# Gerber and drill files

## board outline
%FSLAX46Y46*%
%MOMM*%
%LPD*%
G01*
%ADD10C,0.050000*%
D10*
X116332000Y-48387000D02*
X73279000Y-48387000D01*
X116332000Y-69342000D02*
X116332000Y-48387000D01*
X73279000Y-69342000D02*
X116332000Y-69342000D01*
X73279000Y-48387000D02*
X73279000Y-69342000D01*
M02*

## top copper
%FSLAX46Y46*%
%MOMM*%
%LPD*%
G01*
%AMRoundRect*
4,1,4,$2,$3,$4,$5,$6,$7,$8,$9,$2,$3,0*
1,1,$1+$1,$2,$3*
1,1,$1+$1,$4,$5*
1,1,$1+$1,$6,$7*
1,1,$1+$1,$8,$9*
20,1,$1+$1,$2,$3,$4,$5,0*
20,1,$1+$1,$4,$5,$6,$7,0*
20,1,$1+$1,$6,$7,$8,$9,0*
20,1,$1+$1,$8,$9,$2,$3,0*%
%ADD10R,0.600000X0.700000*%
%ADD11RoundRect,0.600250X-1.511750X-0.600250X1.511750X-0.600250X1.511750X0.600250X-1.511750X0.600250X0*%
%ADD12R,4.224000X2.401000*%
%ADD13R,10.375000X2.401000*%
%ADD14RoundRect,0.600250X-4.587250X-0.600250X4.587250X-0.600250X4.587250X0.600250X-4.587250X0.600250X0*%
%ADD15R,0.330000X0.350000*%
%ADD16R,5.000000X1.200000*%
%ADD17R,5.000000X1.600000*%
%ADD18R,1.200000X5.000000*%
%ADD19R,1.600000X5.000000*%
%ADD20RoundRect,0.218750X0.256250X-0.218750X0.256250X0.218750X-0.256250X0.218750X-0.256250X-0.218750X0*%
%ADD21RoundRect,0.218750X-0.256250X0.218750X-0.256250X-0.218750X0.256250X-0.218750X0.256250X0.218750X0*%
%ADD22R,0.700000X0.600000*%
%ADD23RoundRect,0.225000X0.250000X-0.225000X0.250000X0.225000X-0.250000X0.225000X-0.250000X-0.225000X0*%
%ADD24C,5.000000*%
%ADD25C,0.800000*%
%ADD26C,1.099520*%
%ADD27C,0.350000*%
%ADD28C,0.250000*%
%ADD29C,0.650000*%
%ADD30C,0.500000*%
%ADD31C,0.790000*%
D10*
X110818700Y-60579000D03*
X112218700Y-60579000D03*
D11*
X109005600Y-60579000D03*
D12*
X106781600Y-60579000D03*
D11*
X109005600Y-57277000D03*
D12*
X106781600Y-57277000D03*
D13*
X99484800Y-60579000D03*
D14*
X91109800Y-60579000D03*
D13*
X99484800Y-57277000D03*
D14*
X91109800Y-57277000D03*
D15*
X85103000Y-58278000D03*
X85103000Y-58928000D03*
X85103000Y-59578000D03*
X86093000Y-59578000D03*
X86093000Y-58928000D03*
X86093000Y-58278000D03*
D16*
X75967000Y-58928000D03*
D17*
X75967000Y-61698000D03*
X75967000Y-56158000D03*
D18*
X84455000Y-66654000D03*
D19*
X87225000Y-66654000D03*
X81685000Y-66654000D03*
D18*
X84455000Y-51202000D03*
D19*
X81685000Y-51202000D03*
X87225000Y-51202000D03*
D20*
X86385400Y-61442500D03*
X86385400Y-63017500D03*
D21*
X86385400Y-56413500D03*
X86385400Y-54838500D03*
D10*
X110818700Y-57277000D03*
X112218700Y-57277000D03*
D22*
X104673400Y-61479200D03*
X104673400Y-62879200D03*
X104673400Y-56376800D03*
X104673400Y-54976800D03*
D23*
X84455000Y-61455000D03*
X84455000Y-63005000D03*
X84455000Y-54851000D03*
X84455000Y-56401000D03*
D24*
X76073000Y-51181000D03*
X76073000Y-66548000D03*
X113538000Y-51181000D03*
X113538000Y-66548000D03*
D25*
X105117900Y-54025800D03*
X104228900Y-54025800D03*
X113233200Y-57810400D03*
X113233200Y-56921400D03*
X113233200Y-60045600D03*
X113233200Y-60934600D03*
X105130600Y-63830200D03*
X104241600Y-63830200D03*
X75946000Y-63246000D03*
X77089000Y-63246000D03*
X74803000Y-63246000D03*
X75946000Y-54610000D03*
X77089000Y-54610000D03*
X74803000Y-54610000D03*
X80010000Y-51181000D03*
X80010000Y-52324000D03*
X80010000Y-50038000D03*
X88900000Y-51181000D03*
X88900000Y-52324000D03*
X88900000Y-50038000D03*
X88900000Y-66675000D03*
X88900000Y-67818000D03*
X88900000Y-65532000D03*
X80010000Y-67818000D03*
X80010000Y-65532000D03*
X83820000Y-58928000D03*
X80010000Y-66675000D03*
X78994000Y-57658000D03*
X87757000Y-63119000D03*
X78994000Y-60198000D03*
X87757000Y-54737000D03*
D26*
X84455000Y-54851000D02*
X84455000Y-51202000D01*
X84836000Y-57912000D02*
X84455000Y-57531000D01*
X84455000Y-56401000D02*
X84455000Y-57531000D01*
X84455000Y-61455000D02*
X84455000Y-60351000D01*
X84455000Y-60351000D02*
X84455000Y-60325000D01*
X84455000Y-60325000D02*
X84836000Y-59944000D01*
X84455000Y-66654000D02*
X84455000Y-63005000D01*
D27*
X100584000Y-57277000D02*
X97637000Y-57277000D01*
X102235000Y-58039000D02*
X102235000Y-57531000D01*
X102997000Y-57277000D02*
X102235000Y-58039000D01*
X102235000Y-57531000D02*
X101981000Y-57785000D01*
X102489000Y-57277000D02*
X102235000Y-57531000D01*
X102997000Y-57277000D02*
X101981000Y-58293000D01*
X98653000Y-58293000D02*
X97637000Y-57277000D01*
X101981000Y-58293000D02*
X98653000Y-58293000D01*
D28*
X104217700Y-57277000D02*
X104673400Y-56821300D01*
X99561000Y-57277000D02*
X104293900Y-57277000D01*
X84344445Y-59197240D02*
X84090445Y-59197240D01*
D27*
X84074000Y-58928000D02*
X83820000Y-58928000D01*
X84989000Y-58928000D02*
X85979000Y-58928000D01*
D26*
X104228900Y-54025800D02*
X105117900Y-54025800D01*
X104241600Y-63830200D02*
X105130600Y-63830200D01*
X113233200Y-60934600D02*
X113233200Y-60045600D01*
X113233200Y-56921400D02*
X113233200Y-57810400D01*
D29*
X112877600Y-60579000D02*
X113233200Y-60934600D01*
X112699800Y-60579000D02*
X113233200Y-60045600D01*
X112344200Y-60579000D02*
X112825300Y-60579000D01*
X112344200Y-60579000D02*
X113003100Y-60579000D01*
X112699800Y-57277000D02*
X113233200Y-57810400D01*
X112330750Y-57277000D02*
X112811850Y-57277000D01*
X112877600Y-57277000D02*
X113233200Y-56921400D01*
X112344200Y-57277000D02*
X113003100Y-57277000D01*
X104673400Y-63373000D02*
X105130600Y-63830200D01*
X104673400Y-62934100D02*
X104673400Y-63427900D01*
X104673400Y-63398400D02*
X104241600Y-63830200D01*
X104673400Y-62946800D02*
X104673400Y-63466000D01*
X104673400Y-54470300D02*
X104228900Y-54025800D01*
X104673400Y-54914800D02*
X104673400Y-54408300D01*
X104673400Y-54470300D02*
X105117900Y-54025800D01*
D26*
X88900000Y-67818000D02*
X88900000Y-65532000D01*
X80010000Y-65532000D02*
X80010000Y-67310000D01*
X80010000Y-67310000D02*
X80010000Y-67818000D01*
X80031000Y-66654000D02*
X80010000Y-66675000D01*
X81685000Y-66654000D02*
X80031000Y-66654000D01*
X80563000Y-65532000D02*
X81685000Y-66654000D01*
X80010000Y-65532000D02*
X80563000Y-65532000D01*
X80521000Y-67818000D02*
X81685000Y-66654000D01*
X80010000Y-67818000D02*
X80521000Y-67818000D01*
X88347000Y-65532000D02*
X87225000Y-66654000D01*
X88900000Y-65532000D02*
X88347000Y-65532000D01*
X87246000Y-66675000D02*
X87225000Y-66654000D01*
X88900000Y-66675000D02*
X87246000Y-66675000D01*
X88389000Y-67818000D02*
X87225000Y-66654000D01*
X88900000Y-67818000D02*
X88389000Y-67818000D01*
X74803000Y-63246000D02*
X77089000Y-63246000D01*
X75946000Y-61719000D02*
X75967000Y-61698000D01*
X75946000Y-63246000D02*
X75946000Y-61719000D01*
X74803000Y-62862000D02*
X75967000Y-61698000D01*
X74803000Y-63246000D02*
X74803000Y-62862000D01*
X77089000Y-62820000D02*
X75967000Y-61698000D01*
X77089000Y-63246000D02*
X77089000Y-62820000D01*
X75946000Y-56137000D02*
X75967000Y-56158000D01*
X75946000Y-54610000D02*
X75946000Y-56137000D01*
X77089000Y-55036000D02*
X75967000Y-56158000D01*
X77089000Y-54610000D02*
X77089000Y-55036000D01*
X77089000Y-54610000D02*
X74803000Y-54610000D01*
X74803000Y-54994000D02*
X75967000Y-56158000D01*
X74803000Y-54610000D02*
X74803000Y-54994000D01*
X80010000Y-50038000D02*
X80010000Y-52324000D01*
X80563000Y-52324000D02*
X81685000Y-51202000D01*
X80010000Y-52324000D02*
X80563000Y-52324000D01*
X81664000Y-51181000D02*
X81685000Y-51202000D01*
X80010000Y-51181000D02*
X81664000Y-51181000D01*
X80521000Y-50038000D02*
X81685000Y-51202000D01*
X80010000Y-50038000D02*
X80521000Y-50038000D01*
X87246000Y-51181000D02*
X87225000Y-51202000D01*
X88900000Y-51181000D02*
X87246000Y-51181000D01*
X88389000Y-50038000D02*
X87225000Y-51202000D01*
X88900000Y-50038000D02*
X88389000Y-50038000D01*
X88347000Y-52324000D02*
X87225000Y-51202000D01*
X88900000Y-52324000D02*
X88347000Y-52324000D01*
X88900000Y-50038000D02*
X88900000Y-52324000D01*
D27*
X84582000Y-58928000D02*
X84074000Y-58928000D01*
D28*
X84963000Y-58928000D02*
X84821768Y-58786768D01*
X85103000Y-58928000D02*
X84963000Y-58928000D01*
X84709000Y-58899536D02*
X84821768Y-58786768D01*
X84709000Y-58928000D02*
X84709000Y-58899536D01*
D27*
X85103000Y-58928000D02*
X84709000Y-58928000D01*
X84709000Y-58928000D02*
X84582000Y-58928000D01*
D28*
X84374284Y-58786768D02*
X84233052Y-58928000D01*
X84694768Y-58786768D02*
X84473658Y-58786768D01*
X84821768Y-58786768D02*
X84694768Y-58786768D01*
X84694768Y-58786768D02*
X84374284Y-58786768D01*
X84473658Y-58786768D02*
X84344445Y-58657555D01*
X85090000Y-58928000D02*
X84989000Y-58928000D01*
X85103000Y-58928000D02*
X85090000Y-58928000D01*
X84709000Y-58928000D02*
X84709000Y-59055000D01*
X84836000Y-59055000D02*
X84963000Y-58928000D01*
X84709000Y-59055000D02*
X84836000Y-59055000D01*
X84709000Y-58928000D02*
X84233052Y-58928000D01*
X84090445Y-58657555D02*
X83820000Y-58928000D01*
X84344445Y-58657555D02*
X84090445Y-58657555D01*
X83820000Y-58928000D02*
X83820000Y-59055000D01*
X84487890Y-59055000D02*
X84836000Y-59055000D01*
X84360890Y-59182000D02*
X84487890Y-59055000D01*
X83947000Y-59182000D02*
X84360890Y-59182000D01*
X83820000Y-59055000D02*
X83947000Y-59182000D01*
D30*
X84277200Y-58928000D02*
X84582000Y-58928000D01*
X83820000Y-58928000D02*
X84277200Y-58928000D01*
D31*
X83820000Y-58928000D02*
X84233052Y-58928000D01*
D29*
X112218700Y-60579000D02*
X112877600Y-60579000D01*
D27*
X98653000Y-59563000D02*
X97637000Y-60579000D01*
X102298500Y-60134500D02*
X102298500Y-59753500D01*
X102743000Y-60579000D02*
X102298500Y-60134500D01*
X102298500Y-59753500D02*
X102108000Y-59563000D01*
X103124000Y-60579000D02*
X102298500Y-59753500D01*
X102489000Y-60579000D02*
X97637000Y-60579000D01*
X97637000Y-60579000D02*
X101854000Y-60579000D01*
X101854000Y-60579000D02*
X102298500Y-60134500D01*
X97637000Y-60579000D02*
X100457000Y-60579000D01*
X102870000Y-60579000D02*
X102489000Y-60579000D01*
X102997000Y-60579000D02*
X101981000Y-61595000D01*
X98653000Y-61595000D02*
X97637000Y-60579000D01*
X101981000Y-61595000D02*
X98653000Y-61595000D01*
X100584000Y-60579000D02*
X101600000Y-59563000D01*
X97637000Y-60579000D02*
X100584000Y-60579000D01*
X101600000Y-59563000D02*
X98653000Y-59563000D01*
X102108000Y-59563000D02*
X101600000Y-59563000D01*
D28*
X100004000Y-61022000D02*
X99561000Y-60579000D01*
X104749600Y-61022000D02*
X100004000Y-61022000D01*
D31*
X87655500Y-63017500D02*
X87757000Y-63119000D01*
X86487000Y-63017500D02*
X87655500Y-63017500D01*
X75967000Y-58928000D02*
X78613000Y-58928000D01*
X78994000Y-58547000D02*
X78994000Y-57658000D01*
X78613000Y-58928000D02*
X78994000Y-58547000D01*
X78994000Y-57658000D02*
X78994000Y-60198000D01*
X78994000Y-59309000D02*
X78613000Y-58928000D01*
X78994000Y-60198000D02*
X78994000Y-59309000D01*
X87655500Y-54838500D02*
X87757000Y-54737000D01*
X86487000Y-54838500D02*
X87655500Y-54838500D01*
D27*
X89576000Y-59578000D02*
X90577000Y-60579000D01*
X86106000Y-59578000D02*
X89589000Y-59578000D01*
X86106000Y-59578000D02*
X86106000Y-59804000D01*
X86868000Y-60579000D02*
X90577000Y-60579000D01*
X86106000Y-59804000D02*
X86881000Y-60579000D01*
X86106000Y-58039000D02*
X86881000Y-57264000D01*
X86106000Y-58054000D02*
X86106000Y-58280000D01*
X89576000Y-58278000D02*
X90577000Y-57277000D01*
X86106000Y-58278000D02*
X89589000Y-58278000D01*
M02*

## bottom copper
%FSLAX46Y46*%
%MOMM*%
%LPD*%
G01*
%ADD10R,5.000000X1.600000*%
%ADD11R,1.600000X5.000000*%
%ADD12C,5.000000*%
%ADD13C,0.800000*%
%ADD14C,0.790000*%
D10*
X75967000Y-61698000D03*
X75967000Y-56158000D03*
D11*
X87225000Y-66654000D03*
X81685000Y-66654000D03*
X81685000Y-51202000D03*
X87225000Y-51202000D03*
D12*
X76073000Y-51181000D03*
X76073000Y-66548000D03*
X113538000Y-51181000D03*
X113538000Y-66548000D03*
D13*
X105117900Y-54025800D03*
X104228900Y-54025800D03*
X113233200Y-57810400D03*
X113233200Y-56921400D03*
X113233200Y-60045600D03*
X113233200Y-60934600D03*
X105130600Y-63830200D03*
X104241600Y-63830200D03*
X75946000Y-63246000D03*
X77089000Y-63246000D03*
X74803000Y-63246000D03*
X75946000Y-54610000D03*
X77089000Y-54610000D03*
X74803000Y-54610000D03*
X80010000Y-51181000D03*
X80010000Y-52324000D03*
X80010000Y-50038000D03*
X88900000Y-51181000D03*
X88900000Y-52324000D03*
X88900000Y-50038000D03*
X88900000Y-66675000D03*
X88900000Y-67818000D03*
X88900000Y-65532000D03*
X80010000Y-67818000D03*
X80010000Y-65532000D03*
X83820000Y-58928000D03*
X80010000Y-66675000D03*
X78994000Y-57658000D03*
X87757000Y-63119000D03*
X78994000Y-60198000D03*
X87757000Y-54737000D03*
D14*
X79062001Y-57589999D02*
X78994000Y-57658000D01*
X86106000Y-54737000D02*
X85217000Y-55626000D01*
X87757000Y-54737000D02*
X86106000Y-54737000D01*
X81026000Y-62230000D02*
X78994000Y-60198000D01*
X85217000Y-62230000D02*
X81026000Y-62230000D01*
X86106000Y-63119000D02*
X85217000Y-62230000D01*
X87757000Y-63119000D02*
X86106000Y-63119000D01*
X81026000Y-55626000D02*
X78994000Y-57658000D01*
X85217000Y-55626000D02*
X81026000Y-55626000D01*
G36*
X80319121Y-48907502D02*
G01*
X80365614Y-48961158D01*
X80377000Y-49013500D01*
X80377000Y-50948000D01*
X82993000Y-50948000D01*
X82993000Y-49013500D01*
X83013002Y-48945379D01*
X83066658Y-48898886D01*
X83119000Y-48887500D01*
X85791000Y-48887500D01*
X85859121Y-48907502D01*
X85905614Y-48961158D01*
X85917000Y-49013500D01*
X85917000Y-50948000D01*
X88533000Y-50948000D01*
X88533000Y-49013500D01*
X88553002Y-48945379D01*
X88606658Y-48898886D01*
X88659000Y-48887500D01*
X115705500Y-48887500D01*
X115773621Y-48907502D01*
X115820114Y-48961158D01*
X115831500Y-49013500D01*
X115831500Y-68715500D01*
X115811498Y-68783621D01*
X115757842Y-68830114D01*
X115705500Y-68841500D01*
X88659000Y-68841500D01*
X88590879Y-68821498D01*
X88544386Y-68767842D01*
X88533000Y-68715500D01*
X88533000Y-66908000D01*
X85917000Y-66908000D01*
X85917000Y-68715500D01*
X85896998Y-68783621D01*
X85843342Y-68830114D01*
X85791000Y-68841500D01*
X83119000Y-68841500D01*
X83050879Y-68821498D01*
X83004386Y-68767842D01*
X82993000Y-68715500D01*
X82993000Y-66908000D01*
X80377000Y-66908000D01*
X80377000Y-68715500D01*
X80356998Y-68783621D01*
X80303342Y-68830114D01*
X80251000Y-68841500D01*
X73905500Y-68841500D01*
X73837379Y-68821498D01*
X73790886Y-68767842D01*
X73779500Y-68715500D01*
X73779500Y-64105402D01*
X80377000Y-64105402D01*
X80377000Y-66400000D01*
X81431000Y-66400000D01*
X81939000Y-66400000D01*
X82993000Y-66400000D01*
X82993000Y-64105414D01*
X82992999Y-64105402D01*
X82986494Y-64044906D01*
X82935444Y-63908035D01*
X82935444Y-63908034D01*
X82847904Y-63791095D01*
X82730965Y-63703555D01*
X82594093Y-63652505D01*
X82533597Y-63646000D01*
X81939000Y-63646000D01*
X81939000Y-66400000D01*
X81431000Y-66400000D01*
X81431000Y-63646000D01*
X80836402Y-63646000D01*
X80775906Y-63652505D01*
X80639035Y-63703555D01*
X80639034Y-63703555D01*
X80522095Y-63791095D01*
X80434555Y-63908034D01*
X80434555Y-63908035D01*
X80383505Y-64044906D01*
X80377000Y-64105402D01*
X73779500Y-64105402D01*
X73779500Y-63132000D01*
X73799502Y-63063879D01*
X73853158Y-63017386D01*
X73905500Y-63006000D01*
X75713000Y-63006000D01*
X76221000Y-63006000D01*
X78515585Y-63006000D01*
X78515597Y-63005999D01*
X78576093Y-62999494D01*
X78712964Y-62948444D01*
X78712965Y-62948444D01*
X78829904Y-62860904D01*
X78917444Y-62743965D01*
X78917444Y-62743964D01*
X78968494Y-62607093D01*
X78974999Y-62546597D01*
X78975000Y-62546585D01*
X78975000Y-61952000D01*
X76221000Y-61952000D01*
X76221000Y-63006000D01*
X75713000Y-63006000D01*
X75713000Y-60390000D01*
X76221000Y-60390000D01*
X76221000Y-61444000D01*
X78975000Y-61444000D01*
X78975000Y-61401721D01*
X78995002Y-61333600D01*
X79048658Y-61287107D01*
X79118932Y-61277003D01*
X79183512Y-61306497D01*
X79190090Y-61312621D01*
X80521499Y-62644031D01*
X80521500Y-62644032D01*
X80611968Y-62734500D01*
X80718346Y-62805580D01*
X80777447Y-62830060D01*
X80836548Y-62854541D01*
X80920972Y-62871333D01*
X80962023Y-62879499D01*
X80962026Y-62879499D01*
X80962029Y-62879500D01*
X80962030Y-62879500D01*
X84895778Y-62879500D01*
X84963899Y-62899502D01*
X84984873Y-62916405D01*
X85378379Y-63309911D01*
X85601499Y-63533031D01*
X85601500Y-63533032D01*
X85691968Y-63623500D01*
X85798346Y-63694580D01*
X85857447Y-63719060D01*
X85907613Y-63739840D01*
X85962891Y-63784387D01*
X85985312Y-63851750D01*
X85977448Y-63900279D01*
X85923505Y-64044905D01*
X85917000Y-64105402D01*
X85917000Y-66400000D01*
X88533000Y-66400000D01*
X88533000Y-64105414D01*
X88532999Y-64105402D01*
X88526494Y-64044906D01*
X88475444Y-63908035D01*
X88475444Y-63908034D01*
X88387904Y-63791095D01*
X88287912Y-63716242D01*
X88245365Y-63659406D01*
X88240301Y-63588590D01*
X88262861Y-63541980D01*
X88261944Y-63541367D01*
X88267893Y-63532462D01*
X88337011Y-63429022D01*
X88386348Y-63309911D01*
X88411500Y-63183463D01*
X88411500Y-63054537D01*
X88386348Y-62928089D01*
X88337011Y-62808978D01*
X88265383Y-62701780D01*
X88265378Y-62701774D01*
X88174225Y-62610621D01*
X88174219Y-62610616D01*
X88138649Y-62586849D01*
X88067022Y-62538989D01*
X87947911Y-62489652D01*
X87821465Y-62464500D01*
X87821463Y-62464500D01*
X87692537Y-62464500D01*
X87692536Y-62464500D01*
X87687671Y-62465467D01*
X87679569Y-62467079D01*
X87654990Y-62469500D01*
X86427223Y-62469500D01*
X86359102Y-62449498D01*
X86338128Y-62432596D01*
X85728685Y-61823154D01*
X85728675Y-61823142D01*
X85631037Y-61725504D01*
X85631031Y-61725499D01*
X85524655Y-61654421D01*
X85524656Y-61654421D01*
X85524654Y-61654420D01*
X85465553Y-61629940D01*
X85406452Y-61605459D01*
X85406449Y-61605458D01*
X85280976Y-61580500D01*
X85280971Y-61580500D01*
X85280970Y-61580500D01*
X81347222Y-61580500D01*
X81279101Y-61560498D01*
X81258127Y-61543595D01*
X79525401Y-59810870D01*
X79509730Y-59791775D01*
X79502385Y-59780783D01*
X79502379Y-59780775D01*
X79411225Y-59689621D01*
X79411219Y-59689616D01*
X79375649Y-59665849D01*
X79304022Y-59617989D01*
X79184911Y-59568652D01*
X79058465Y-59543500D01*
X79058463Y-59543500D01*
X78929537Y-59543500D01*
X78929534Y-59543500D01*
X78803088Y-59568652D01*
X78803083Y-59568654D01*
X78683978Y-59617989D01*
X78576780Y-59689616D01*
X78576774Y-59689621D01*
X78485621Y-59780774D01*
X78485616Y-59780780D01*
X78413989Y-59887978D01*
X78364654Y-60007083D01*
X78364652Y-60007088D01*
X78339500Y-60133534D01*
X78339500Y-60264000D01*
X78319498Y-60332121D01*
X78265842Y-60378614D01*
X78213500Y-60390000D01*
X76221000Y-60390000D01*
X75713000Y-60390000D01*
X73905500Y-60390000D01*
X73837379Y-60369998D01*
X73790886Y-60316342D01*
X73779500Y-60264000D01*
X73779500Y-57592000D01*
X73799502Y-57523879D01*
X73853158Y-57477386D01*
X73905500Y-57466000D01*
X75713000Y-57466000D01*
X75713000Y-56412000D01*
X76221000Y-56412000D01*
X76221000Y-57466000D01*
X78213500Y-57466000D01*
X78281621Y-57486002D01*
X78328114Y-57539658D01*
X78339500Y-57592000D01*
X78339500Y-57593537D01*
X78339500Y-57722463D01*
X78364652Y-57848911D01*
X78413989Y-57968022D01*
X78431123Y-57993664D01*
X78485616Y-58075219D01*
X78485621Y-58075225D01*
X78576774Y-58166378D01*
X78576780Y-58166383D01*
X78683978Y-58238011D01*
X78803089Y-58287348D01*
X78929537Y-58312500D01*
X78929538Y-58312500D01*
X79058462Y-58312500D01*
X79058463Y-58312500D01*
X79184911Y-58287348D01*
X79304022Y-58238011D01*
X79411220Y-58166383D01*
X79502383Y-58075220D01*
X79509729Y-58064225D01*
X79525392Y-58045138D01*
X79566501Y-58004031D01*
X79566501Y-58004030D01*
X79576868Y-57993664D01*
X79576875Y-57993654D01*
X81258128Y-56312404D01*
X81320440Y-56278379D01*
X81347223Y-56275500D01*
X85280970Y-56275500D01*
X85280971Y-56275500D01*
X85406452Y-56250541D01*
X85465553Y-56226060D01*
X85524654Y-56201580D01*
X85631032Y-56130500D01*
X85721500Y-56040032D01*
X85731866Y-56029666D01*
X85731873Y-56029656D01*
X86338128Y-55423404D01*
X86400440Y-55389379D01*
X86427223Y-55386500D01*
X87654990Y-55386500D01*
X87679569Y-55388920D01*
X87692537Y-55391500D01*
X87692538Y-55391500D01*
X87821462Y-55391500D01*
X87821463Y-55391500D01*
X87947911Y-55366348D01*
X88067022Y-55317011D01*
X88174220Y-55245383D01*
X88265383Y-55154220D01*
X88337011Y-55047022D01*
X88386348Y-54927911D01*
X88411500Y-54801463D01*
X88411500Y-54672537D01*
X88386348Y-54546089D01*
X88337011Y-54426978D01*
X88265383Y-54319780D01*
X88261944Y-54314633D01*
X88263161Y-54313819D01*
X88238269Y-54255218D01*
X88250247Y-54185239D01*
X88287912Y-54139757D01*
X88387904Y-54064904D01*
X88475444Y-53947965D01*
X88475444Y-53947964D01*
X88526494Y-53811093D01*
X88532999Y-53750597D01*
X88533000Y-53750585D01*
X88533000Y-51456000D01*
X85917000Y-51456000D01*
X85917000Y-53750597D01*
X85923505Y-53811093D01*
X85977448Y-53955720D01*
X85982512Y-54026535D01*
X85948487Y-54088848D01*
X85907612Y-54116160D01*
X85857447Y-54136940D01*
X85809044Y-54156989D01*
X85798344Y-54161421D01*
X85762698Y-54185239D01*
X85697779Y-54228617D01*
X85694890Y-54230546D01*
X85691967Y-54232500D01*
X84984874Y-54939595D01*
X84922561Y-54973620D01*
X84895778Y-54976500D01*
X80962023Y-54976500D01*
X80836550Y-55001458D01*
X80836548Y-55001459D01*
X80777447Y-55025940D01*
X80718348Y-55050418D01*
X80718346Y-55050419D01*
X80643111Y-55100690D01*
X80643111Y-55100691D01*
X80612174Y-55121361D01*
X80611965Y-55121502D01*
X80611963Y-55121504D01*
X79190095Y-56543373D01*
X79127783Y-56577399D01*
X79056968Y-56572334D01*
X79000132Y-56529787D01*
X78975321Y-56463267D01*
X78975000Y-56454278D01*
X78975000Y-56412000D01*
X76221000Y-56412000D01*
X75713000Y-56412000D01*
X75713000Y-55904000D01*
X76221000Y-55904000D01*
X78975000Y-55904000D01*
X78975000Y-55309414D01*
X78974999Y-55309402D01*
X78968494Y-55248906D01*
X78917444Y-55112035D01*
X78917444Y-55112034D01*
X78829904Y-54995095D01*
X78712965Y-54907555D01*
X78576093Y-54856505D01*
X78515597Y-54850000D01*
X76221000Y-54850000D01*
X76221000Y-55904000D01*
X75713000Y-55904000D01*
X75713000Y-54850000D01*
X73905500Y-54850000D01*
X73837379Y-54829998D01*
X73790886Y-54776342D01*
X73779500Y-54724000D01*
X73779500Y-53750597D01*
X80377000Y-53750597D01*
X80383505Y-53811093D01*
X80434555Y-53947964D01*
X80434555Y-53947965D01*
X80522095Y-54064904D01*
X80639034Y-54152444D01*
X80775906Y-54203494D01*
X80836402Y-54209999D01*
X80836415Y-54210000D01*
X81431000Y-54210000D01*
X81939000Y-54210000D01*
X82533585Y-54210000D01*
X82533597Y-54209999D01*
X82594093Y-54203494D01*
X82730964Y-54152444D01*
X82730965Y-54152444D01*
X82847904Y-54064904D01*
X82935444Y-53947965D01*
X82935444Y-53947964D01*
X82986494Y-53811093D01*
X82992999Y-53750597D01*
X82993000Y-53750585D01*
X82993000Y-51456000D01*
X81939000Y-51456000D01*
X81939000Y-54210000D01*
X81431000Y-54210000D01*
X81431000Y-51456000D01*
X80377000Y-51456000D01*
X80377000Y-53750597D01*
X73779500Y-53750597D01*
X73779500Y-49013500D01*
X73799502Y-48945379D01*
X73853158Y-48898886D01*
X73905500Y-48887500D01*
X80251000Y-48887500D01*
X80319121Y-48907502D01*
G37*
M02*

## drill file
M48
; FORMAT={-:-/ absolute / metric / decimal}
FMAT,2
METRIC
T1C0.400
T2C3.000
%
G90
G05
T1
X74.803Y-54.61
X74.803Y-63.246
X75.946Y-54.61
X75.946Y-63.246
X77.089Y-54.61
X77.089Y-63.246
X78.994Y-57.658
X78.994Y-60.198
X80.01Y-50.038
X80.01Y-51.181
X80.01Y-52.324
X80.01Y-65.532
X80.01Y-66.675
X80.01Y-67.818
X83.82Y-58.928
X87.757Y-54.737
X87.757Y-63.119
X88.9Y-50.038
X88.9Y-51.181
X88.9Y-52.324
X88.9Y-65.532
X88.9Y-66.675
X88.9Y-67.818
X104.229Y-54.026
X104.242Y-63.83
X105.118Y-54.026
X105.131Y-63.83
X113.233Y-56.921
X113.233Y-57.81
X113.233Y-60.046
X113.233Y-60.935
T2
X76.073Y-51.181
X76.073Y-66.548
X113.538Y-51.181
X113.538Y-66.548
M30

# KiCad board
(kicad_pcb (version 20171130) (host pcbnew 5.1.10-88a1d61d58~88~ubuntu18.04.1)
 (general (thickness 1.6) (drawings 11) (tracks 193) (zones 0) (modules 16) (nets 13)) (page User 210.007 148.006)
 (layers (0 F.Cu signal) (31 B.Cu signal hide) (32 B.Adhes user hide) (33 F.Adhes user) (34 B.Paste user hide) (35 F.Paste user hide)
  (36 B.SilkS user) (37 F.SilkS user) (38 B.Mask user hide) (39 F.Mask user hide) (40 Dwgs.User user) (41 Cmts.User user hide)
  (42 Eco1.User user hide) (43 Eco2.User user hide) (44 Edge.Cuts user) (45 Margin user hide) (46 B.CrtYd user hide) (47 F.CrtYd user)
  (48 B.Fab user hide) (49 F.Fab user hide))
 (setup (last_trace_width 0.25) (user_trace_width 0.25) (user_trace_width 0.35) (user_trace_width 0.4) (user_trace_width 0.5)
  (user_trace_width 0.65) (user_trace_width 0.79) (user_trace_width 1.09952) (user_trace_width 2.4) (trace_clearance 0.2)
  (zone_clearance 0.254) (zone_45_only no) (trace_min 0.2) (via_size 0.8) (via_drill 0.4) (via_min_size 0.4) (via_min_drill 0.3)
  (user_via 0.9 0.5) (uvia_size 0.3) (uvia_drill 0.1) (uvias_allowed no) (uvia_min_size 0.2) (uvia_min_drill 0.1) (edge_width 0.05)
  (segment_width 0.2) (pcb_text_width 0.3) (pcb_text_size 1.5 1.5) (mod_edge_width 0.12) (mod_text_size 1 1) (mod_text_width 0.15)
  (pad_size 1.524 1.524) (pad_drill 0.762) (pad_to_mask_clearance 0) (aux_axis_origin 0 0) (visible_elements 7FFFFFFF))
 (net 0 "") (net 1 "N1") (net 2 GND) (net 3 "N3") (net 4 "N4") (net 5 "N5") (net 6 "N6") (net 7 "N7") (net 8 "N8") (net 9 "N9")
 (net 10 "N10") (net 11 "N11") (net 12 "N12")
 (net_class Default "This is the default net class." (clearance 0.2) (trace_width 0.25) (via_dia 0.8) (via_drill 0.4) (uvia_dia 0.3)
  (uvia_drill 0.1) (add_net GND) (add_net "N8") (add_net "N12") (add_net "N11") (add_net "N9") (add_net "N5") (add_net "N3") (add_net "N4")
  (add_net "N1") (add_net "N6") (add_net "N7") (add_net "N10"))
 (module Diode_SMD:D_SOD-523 (layer F.Cu) (at 111.5187 60.579)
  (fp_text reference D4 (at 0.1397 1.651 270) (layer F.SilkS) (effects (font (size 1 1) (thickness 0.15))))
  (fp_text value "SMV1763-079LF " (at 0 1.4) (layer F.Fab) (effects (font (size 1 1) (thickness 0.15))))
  (pad 1 smd rect (at -0.7 0 180) (size 0.6 0.7) (layers F.Cu F.Paste F.Mask) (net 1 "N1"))
  (pad 2 smd rect (at 0.7 0 180) (size 0.6 0.7) (layers F.Cu F.Paste F.Mask) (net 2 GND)))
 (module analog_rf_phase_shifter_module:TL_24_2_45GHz (layer F.Cu) (at 107.8936 60.579)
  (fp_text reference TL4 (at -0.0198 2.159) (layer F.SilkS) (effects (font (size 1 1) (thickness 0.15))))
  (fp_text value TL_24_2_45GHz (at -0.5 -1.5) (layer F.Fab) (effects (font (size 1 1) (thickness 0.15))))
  (pad 2 smd roundrect (at 1.112 0) (size 4.224 2.401) (layers F.Cu) (roundrect_rratio 0.25) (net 1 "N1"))
  (pad 1 smd rect (at -1.112 0) (size 4.224 2.401) (layers F.Cu) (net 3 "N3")))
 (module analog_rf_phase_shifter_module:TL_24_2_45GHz (layer F.Cu) (at 107.8936 57.277)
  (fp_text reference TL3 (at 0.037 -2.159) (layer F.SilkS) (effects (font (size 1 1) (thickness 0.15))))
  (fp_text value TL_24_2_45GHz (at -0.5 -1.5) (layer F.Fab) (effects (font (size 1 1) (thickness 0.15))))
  (pad 2 smd roundrect (at 1.112 0) (size 4.224 2.401) (layers F.Cu) (roundrect_rratio 0.25) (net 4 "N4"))
  (pad 1 smd rect (at -1.112 0) (size 4.224 2.401) (layers F.Cu) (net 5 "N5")))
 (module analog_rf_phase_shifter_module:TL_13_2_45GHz (layer F.Cu) (at 95.2973 60.579)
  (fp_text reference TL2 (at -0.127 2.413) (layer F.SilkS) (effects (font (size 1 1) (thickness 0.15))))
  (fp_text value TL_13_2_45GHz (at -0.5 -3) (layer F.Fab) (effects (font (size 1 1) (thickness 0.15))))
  (pad 2 smd rect (at 4.1875 0) (size 10.375 2.401) (layers F.Cu) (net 3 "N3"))
  (pad 1 smd roundrect (at -4.1875 0) (size 10.375 2.401) (layers F.Cu) (roundrect_rratio 0.25) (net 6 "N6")))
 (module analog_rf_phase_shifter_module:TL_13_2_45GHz (layer F.Cu) (at 95.2973 57.277)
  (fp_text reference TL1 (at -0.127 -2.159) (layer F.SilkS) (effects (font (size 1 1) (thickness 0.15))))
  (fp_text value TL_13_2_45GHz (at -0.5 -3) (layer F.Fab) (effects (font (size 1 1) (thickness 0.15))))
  (pad 2 smd rect (at 4.1875 0) (size 10.375 2.401) (layers F.Cu) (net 5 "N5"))
  (pad 1 smd roundrect (at -4.1875 0) (size 10.375 2.401) (layers F.Cu) (roundrect_rratio 0.25) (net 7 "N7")))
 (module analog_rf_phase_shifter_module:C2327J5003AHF (layer F.Cu) (at 85.598 58.928 270)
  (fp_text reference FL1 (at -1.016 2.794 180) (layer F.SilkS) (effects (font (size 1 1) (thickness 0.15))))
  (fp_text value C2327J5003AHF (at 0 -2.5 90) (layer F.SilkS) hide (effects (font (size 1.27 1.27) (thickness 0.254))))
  (pad 1 smd rect (at -0.65 0.495) (size 0.33 0.35) (layers F.Cu F.Paste F.Mask) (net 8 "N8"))
  (pad 2 smd rect (at 0 0.495) (size 0.33 0.35) (layers F.Cu F.Paste F.Mask) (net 2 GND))
  (pad 3 smd rect (at 0.65 0.495) (size 0.33 0.35) (layers F.Cu F.Paste F.Mask) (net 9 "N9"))
  (pad 4 smd rect (at 0.65 -0.495) (size 0.33 0.35) (layers F.Cu F.Paste F.Mask) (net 6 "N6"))
  (pad 5 smd rect (at 0 -0.495) (size 0.33 0.35) (layers F.Cu F.Paste F.Mask) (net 2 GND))
  (pad 6 smd rect (at -0.65 -0.495) (size 0.33 0.35) (layers F.Cu F.Paste F.Mask) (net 7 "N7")))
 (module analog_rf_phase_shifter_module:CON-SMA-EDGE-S (layer F.Cu) (at 68.707 58.928 90)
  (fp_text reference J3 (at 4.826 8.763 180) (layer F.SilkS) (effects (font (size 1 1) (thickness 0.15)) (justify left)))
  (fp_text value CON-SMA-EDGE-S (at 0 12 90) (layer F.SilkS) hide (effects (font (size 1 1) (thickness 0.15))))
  (pad 1 smd rect (at 0 7.26 90) (size 1.2 5) (layers F.Cu F.Paste F.Mask) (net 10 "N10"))
  (pad 2 smd rect (at -2.77 7.26 90) (size 1.6 5) (layers F.Cu F.Paste F.Mask) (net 2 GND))
  (pad 2 smd rect (at 2.77 7.26 90) (size 1.6 5) (layers F.Cu F.Paste F.Mask) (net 2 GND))
  (pad 2 smd rect (at -2.77 7.26 90) (size 1.6 5) (layers B.Cu B.Paste B.Mask) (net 2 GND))
  (pad 2 smd rect (at 2.77 7.26 90) (size 1.6 5) (layers B.Cu B.Paste B.Mask) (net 2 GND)))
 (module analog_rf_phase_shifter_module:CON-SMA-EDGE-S (layer F.Cu) (at 84.455 73.914 180)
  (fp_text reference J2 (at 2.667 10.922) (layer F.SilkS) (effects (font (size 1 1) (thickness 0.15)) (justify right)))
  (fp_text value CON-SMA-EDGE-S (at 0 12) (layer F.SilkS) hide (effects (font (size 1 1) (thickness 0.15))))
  (pad 1 smd rect (at 0 7.26 180) (size 1.2 5) (layers F.Cu F.Paste F.Mask) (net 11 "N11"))
  (pad 2 smd rect (at -2.77 7.26 180) (size 1.6 5) (layers F.Cu F.Paste F.Mask) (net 2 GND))
  (pad 2 smd rect (at 2.77 7.26 180) (size 1.6 5) (layers F.Cu F.Paste F.Mask) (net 2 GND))
  (pad 2 smd rect (at -2.77 7.26 180) (size 1.6 5) (layers B.Cu B.Paste B.Mask) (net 2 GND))
  (pad 2 smd rect (at 2.77 7.26 180) (size 1.6 5) (layers B.Cu B.Paste B.Mask) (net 2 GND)))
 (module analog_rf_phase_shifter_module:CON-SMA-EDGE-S (layer F.Cu) (at 84.455 43.942)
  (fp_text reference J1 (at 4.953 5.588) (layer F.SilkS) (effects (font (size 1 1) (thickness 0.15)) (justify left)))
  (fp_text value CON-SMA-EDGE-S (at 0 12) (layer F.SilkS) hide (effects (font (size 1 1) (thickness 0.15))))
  (pad 1 smd rect (at 0 7.26) (size 1.2 5) (layers F.Cu F.Paste F.Mask) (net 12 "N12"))
  (pad 2 smd rect (at -2.77 7.26) (size 1.6 5) (layers F.Cu F.Paste F.Mask) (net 2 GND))
  (pad 2 smd rect (at 2.77 7.26) (size 1.6 5) (layers F.Cu F.Paste F.Mask) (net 2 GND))
  (pad 2 smd rect (at -2.77 7.26) (size 1.6 5) (layers B.Cu B.Paste B.Mask) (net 2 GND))
  (pad 2 smd rect (at 2.77 7.26) (size 1.6 5) (layers B.Cu B.Paste B.Mask) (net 2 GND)))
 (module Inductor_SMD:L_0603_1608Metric (layer F.Cu) (at 86.3854 62.23 90)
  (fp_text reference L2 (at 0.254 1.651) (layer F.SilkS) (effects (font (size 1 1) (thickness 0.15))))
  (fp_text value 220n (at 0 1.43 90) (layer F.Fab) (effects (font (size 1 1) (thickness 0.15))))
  (pad 2 smd roundrect (at 0.7875 0 90) (size 0.875 0.95) (layers F.Cu F.Paste F.Mask) (roundrect_rratio 0.25) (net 6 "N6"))
  (pad 1 smd roundrect (at -0.7875 0 90) (size 0.875 0.95) (layers F.Cu F.Paste F.Mask) (roundrect_rratio 0.25) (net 10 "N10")))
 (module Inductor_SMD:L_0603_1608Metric (layer F.Cu) (at 86.3854 55.626 270)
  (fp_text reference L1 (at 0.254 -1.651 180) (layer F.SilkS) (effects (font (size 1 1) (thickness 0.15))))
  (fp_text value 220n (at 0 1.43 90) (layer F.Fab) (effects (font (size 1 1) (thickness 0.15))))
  (pad 2 smd roundrect (at 0.7875 0 270) (size 0.875 0.95) (layers F.Cu F.Paste F.Mask) (roundrect_rratio 0.25) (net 7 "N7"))
  (pad 1 smd roundrect (at -0.7875 0 270) (size 0.875 0.95) (layers F.Cu F.Paste F.Mask) (roundrect_rratio 0.25) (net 10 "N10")))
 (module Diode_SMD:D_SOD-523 (layer F.Cu) (at 111.5187 57.277)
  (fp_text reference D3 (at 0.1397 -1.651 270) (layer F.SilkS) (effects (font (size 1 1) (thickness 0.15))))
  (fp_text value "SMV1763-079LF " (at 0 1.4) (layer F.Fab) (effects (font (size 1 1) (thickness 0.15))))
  (pad 1 smd rect (at -0.7 0 180) (size 0.6 0.7) (layers F.Cu F.Paste F.Mask) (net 4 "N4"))
  (pad 2 smd rect (at 0.7 0 180) (size 0.6 0.7) (layers F.Cu F.Paste F.Mask) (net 2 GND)))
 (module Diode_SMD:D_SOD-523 (layer F.Cu) (at 104.6734 62.1792 270)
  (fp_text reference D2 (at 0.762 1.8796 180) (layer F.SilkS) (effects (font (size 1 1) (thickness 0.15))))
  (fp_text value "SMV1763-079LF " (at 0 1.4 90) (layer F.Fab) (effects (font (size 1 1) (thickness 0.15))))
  (pad 1 smd rect (at -0.7 0 90) (size 0.6 0.7) (layers F.Cu F.Paste F.Mask) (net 3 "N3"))
  (pad 2 smd rect (at 0.7 0 90) (size 0.6 0.7) (layers F.Cu F.Paste F.Mask) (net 2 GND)))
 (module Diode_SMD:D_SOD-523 (layer F.Cu) (at 104.6734 55.6768 90)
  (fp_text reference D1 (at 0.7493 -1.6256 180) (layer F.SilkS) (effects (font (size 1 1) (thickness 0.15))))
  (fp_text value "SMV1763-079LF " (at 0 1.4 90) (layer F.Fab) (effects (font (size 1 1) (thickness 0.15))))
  (pad 1 smd rect (at -0.7 0 270) (size 0.6 0.7) (layers F.Cu F.Paste F.Mask) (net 5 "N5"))
  (pad 2 smd rect (at 0.7 0 270) (size 0.6 0.7) (layers F.Cu F.Paste F.Mask) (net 2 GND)))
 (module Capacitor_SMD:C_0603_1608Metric (layer F.Cu) (at 84.455 62.23 90)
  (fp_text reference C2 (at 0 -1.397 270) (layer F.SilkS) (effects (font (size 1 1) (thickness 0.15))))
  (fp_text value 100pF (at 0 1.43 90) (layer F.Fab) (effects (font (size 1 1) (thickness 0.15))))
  (pad 2 smd roundrect (at 0.775 0 90) (size 0.9 0.95) (layers F.Cu F.Paste F.Mask) (roundrect_rratio 0.25) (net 9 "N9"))
  (pad 1 smd roundrect (at -0.775 0 90) (size 0.9 0.95) (layers F.Cu F.Paste F.Mask) (roundrect_rratio 0.25) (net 11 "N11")))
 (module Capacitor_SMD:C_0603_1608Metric (layer F.Cu) (at 84.455 55.626 90)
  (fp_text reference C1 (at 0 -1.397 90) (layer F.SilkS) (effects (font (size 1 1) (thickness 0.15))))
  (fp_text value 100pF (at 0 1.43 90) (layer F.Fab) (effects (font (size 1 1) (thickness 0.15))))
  (pad 2 smd roundrect (at 0.775 0 90) (size 0.9 0.95) (layers F.Cu F.Paste F.Mask) (roundrect_rratio 0.25) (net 12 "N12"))
  (pad 1 smd roundrect (at -0.775 0 90) (size 0.9 0.95) (layers F.Cu F.Paste F.Mask) (roundrect_rratio 0.25) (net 8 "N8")))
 (gr_line (start 116.332 48.387) (end 73.279 48.387) (layer Edge.Cuts) (width 0.05))
 (gr_line (start 116.332 69.342) (end 116.332 48.387) (layer Edge.Cuts) (width 0.05))
 (gr_line (start 73.279 69.342) (end 116.332 69.342) (layer Edge.Cuts) (width 0.05))
 (gr_line (start 73.279 48.387) (end 73.279 69.342) (layer Edge.Cuts) (width 0.05))
 (segment (start 84.455 54.851) (end 84.455 51.202) (width 1.09952) (layer F.Cu) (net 12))
 (segment (start 84.836 57.912) (end 84.455 57.531) (width 1.09952) (layer F.Cu) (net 8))
 (segment (start 84.455 56.401) (end 84.455 57.531) (width 1.09952) (layer F.Cu) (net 8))
 (segment (start 84.455 61.455) (end 84.455 60.351) (width 1.09952) (layer F.Cu) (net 9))
 (segment (start 84.455 60.351) (end 84.455 60.325) (width 1.09952) (layer F.Cu) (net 9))
 (segment (start 84.455 60.325) (end 84.836 59.944) (width 1.09952) (layer F.Cu) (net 9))
 (segment (start 84.455 66.654) (end 84.455 63.005) (width 1.09952) (layer F.Cu) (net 11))
 (segment (start 100.584 57.277) (end 97.637 57.277) (width 0.35) (layer F.Cu) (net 5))
 (segment (start 102.235 58.039) (end 102.235 57.531) (width 0.35) (layer F.Cu) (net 5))
 (segment (start 102.997 57.277) (end 102.235 58.039) (width 0.35) (layer F.Cu) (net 5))
 (segment (start 102.235 57.531) (end 101.981 57.785) (width 0.35) (layer F.Cu) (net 5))
 (segment (start 102.489 57.277) (end 102.235 57.531) (width 0.35) (layer F.Cu) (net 5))
 (segment (start 102.997 57.277) (end 101.981 58.293) (width 0.35) (layer F.Cu) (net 5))
 (segment (start 98.653 58.293) (end 97.637 57.277) (width 0.35) (layer F.Cu) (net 5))
 (segment (start 101.981 58.293) (end 98.653 58.293) (width 0.35) (layer F.Cu) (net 5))
 (segment (start 104.2177 57.277) (end 104.6734 56.8213) (width 0.25) (layer F.Cu) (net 5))
 (segment (start 99.561 57.277) (end 104.2939 57.277) (width 0.25) (layer F.Cu) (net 5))
 (segment (start 84.344445 59.19724) (end 84.090445 59.19724) (width 0.25) (layer F.Cu) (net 2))
 (via (at 76.073 51.181) (size 5) (drill 3) (layers F.Cu B.Cu) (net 2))
 (via (at 76.073 66.548) (size 5) (drill 3) (layers F.Cu B.Cu) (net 2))
 (via (at 113.538 51.181) (size 5) (drill 3) (layers F.Cu B.Cu) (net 2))
 (via (at 113.538 66.548) (size 5) (drill 3) (layers F.Cu B.Cu) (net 2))
 (via (at 105.1179 54.0258) (size 0.8) (drill 0.4) (layers F.Cu B.Cu) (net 2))
 (via (at 104.2289 54.0258) (size 0.8) (drill 0.4) (layers F.Cu B.Cu) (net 2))
 (via (at 113.2332 57.8104) (size 0.8) (drill 0.4) (layers F.Cu B.Cu) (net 2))
 (via (at 113.2332 56.9214) (size 0.8) (drill 0.4) (layers F.Cu B.Cu) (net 2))
 (via (at 113.2332 60.0456) (size 0.8) (drill 0.4) (layers F.Cu B.Cu) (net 2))
 (via (at 113.2332 60.9346) (size 0.8) (drill 0.4) (layers F.Cu B.Cu) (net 2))
 (via (at 105.1306 63.8302) (size 0.8) (drill 0.4) (layers F.Cu B.Cu) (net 2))
 (via (at 104.2416 63.8302) (size 0.8) (drill 0.4) (layers F.Cu B.Cu) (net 2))
 (via (at 75.946 63.246) (size 0.8) (drill 0.4) (layers F.Cu B.Cu) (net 2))
 (via (at 77.089 63.246) (size 0.8) (drill 0.4) (layers F.Cu B.Cu) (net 2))
 (via (at 74.803 63.246) (size 0.8) (drill 0.4) (layers F.Cu B.Cu) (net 2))
 (via (at 75.946 54.61) (size 0.8) (drill 0.4) (layers F.Cu B.Cu) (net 2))
 (via (at 77.089 54.61) (size 0.8) (drill 0.4) (layers F.Cu B.Cu) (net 2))
 (via (at 74.803 54.61) (size 0.8) (drill 0.4) (layers F.Cu B.Cu) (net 2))
 (via (at 80.01 51.181) (size 0.8) (drill 0.4) (layers F.Cu B.Cu) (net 2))
 (via (at 80.01 52.324) (size 0.8) (drill 0.4) (layers F.Cu B.Cu) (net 2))
 (via (at 80.01 50.038) (size 0.8) (drill 0.4) (layers F.Cu B.Cu) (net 2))
 (via (at 88.9 51.181) (size 0.8) (drill 0.4) (layers F.Cu B.Cu) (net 2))
 (via (at 88.9 52.324) (size 0.8) (drill 0.4) (layers F.Cu B.Cu) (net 2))
 (via (at 88.9 50.038) (size 0.8) (drill 0.4) (layers F.Cu B.Cu) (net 2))
 (via (at 88.9 66.675) (size 0.8) (drill 0.4) (layers F.Cu B.Cu) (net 2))
 (via (at 88.9 67.818) (size 0.8) (drill 0.4) (layers F.Cu B.Cu) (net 2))
 (via (at 88.9 65.532) (size 0.8) (drill 0.4) (layers F.Cu B.Cu) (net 2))
 (via (at 80.01 67.818) (size 0.8) (drill 0.4) (layers F.Cu B.Cu) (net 2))
 (via (at 80.01 65.532) (size 0.8) (drill 0.4) (layers F.Cu B.Cu) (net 2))
 (via (at 83.82 58.928) (size 0.8) (drill 0.4) (layers F.Cu B.Cu) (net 2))
 (segment (start 84.074 58.928) (end 83.82 58.928) (width 0.35) (layer F.Cu) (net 2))
 (segment (start 84.989 58.928) (end 85.979 58.928) (width 0.35) (layer F.Cu) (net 2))
 (via (at 80.01 66.675) (size 0.8) (drill 0.4) (layers F.Cu B.Cu) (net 2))
 (segment (start 104.2289 54.0258) (end 105.1179 54.0258) (width 1.09952) (layer F.Cu) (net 2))
 (segment (start 104.2416 63.8302) (end 105.1306 63.8302) (width 1.09952) (layer F.Cu) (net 2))
 (segment (start 113.2332 60.9346) (end 113.2332 60.0456) (width 1.09952) (layer F.Cu) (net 2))
 (segment (start 113.2332 56.9214) (end 113.2332 57.8104) (width 1.09952) (layer F.Cu) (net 2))
 (segment (start 112.8776 60.579) (end 113.2332 60.9346) (width 0.65) (layer F.Cu) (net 2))
 (segment (start 112.6998 60.579) (end 113.2332 60.0456) (width 0.65) (layer F.Cu) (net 2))
 (segment (start 112.3442 60.579) (end 112.8253 60.579) (width 0.65) (layer F.Cu) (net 2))
 (segment (start 112.3442 60.579) (end 113.0031 60.579) (width 0.65) (layer F.Cu) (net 2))
 (segment (start 112.6998 57.277) (end 113.2332 57.8104) (width 0.65) (layer F.Cu) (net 2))
 (segment (start 112.33075 57.277) (end 112.81185 57.277) (width 0.65) (layer F.Cu) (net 2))
 (segment (start 112.8776 57.277) (end 113.2332 56.9214) (width 0.65) (layer F.Cu) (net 2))
 (segment (start 112.3442 57.277) (end 113.0031 57.277) (width 0.65) (layer F.Cu) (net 2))
 (segment (start 104.6734 63.373) (end 105.1306 63.8302) (width 0.65) (layer F.Cu) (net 2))
 (segment (start 104.6734 62.9341) (end 104.6734 63.4279) (width 0.65) (layer F.Cu) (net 2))
 (segment (start 104.6734 63.3984) (end 104.2416 63.8302) (width 0.65) (layer F.Cu) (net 2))
 (segment (start 104.6734 62.9468) (end 104.6734 63.466) (width 0.65) (layer F.Cu) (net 2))
 (segment (start 104.6734 54.4703) (end 104.2289 54.0258) (width 0.65) (layer F.Cu) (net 2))
 (segment (start 104.6734 54.9148) (end 104.6734 54.4083) (width 0.65) (layer F.Cu) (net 2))
 (segment (start 104.6734 54.4703) (end 105.1179 54.0258) (width 0.65) (layer F.Cu) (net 2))
 (segment (start 88.9 67.818) (end 88.9 65.532) (width 1.09952) (layer F.Cu) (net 2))
 (segment (start 80.01 65.532) (end 80.01 67.31) (width 1.09952) (layer F.Cu) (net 2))
 (segment (start 80.01 67.31) (end 80.01 67.818) (width 1.09952) (layer F.Cu) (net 2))
 (segment (start 80.031 66.654) (end 80.01 66.675) (width 1.09952) (layer F.Cu) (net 2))
 (segment (start 81.685 66.654) (end 80.031 66.654) (width 1.09952) (layer F.Cu) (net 2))
 (segment (start 80.563 65.532) (end 81.685 66.654) (width 1.09952) (layer F.Cu) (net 2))
 (segment (start 80.01 65.532) (end 80.563 65.532) (width 1.09952) (layer F.Cu) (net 2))
 (segment (start 80.521 67.818) (end 81.685 66.654) (width 1.09952) (layer F.Cu) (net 2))
 (segment (start 80.01 67.818) (end 80.521 67.818) (width 1.09952) (layer F.Cu) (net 2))
 (segment (start 88.347 65.532) (end 87.225 66.654) (width 1.09952) (layer F.Cu) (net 2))
 (segment (start 88.9 65.532) (end 88.347 65.532) (width 1.09952) (layer F.Cu) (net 2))
 (segment (start 87.246 66.675) (end 87.225 66.654) (width 1.09952) (layer F.Cu) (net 2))
 (segment (start 88.9 66.675) (end 87.246 66.675) (width 1.09952) (layer F.Cu) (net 2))
 (segment (start 88.389 67.818) (end 87.225 66.654) (width 1.09952) (layer F.Cu) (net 2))
 (segment (start 88.9 67.818) (end 88.389 67.818) (width 1.09952) (layer F.Cu) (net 2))
 (segment (start 74.803 63.246) (end 77.089 63.246) (width 1.09952) (layer F.Cu) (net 2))
 (segment (start 75.946 61.719) (end 75.967 61.698) (width 1.09952) (layer F.Cu) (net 2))
 (segment (start 75.946 63.246) (end 75.946 61.719) (width 1.09952) (layer F.Cu) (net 2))
 (segment (start 74.803 62.862) (end 75.967 61.698) (width 1.09952) (layer F.Cu) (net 2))
 (segment (start 74.803 63.246) (end 74.803 62.862) (width 1.09952) (layer F.Cu) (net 2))
 (segment (start 77.089 62.82) (end 75.967 61.698) (width 1.09952) (layer F.Cu) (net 2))
 (segment (start 77.089 63.246) (end 77.089 62.82) (width 1.09952) (layer F.Cu) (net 2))
 (segment (start 75.946 56.137) (end 75.967 56.158) (width 1.09952) (layer F.Cu) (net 2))
 (segment (start 75.946 54.61) (end 75.946 56.137) (width 1.09952) (layer F.Cu) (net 2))
 (segment (start 77.089 55.036) (end 75.967 56.158) (width 1.09952) (layer F.Cu) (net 2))
 (segment (start 77.089 54.61) (end 77.089 55.036) (width 1.09952) (layer F.Cu) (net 2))
 (segment (start 77.089 54.61) (end 74.803 54.61) (width 1.09952) (layer F.Cu) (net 2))
 (segment (start 74.803 54.994) (end 75.967 56.158) (width 1.09952) (layer F.Cu) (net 2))
 (segment (start 74.803 54.61) (end 74.803 54.994) (width 1.09952) (layer F.Cu) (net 2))
 (segment (start 80.01 50.038) (end 80.01 52.324) (width 1.09952) (layer F.Cu) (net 2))
 (segment (start 80.563 52.324) (end 81.685 51.202) (width 1.09952) (layer F.Cu) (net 2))
 (segment (start 80.01 52.324) (end 80.563 52.324) (width 1.09952) (layer F.Cu) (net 2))
 (segment (start 81.664 51.181) (end 81.685 51.202) (width 1.09952) (layer F.Cu) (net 2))
 (segment (start 80.01 51.181) (end 81.664 51.181) (width 1.09952) (layer F.Cu) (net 2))
 (segment (start 80.521 50.038) (end 81.685 51.202) (width 1.09952) (layer F.Cu) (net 2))
 (segment (start 80.01 50.038) (end 80.521 50.038) (width 1.09952) (layer F.Cu) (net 2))
 (segment (start 87.246 51.181) (end 87.225 51.202) (width 1.09952) (layer F.Cu) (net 2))
 (segment (start 88.9 51.181) (end 87.246 51.181) (width 1.09952) (layer F.Cu) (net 2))
 (segment (start 88.389 50.038) (end 87.225 51.202) (width 1.09952) (layer F.Cu) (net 2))
 (segment (start 88.9 50.038) (end 88.389 50.038) (width 1.09952) (layer F.Cu) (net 2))
 (segment (start 88.347 52.324) (end 87.225 51.202) (width 1.09952) (layer F.Cu) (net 2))
 (segment (start 88.9 52.324) (end 88.347 52.324) (width 1.09952) (layer F.Cu) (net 2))
 (segment (start 88.9 50.038) (end 88.9 52.324) (width 1.09952) (layer F.Cu) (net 2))
 (segment (start 84.582 58.928) (end 84.074 58.928) (width 0.35) (layer F.Cu) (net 2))
 (segment (start 84.963 58.928) (end 84.821768 58.786768) (width 0.25) (layer F.Cu) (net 2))
 (segment (start 85.103 58.928) (end 84.963 58.928) (width 0.25) (layer F.Cu) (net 2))
 (segment (start 84.709 58.899536) (end 84.821768 58.786768) (width 0.25) (layer F.Cu) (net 2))
 (segment (start 84.709 58.928) (end 84.709 58.899536) (width 0.25) (layer F.Cu) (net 2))
 (segment (start 85.103 58.928) (end 84.709 58.928) (width 0.35) (layer F.Cu) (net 2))
 (segment (start 84.709 58.928) (end 84.582 58.928) (width 0.35) (layer F.Cu) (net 2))
 (segment (start 84.374284 58.786768) (end 84.233052 58.928) (width 0.25) (layer F.Cu) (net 2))
 (segment (start 84.694768 58.786768) (end 84.473658 58.786768) (width 0.25) (layer F.Cu) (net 2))
 (segment (start 84.821768 58.786768) (end 84.694768 58.786768) (width 0.25) (layer F.Cu) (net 2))
 (segment (start 84.694768 58.786768) (end 84.374284 58.786768) (width 0.25) (layer F.Cu) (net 2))
 (segment (start 84.473658 58.786768) (end 84.344445 58.657555) (width 0.25) (layer F.Cu) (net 2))
 (segment (start 85.09 58.928) (end 84.989 58.928) (width 0.25) (layer F.Cu) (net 2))
 (segment (start 85.103 58.928) (end 85.09 58.928) (width 0.25) (layer F.Cu) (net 2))
 (segment (start 84.709 58.928) (end 84.709 59.055) (width 0.25) (layer F.Cu) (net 2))
 (segment (start 84.836 59.055) (end 84.963 58.928) (width 0.25) (layer F.Cu) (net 2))
 (segment (start 84.709 59.055) (end 84.836 59.055) (width 0.25) (layer F.Cu) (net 2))
 (segment (start 84.709 58.928) (end 84.233052 58.928) (width 0.25) (layer F.Cu) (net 2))
 (segment (start 84.090445 58.657555) (end 83.82 58.928) (width 0.25) (layer F.Cu) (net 2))
 (segment (start 84.344445 58.657555) (end 84.090445 58.657555) (width 0.25) (layer F.Cu) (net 2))
 (segment (start 83.82 58.928) (end 83.82 59.055) (width 0.25) (layer F.Cu) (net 2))
 (segment (start 84.48789 59.055) (end 84.836 59.055) (width 0.25) (layer F.Cu) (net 2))
 (segment (start 84.36089 59.182) (end 84.48789 59.055) (width 0.25) (layer F.Cu) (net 2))
 (segment (start 83.947 59.182) (end 84.36089 59.182) (width 0.25) (layer F.Cu) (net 2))
 (segment (start 83.82 59.055) (end 83.947 59.182) (width 0.25) (layer F.Cu) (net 2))
 (segment (start 84.2772 58.928) (end 84.582 58.928) (width 0.5) (layer F.Cu) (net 2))
 (segment (start 83.82 58.928) (end 84.2772 58.928) (width 0.5) (layer F.Cu) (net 2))
 (segment (start 83.82 58.928) (end 84.233052 58.928) (width 0.79) (layer F.Cu) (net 2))
 (segment (start 112.2187 60.579) (end 112.8776 60.579) (width 0.65) (layer F.Cu) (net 2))
 (segment (start 98.653 59.563) (end 97.637 60.579) (width 0.35) (layer F.Cu) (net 3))
 (segment (start 102.2985 60.1345) (end 102.2985 59.7535) (width 0.35) (layer F.Cu) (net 3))
 (segment (start 102.743 60.579) (end 102.2985 60.1345) (width 0.35) (layer F.Cu) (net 3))
 (segment (start 102.2985 59.7535) (end 102.108 59.563) (width 0.35) (layer F.Cu) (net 3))
 (segment (start 103.124 60.579) (end 102.2985 59.7535) (width 0.35) (layer F.Cu) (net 3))
 (segment (start 102.489 60.579) (end 97.637 60.579) (width 0.35) (layer F.Cu) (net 3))
 (segment (start 97.637 60.579) (end 101.854 60.579) (width 0.35) (layer F.Cu) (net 3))
 (segment (start 101.854 60.579) (end 102.2985 60.1345) (width 0.35) (layer F.Cu) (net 3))
 (segment (start 97.637 60.579) (end 100.457 60.579) (width 0.35) (layer F.Cu) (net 3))
 (segment (start 102.87 60.579) (end 102.489 60.579) (width 0.35) (layer F.Cu) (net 3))
 (segment (start 102.997 60.579) (end 101.981 61.595) (width 0.35) (layer F.Cu) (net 3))
 (segment (start 98.653 61.595) (end 97.637 60.579) (width 0.35) (layer F.Cu) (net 3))
 (segment (start 101.981 61.595) (end 98.653 61.595) (width 0.35) (layer F.Cu) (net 3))
 (segment (start 100.584 60.579) (end 101.6 59.563) (width 0.35) (layer F.Cu) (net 3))
 (segment (start 97.637 60.579) (end 100.584 60.579) (width 0.35) (layer F.Cu) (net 3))
 (segment (start 101.6 59.563) (end 98.653 59.563) (width 0.35) (layer F.Cu) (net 3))
 (segment (start 102.108 59.563) (end 101.6 59.563) (width 0.35) (layer F.Cu) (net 3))
 (segment (start 100.004 61.022) (end 99.561 60.579) (width 0.25) (layer F.Cu) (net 3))
 (segment (start 104.7496 61.022) (end 100.004 61.022) (width 0.25) (layer F.Cu) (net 3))
 (via (at 78.994 57.658) (size 0.8) (drill 0.4) (layers F.Cu B.Cu) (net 10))
 (segment (start 79.062001 57.589999) (end 78.994 57.658) (width 0.79) (layer B.Cu) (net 10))
 (via (at 87.757 63.119) (size 0.8) (drill 0.4) (layers F.Cu B.Cu) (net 10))
 (segment (start 87.6555 63.0175) (end 87.757 63.119) (width 0.79) (layer F.Cu) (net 10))
 (segment (start 86.487 63.0175) (end 87.6555 63.0175) (width 0.79) (layer F.Cu) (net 10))
 (via (at 78.994 60.198) (size 0.8) (drill 0.4) (layers F.Cu B.Cu) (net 10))
 (segment (start 75.967 58.928) (end 78.613 58.928) (width 0.79) (layer F.Cu) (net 10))
 (segment (start 78.994 58.547) (end 78.994 57.658) (width 0.79) (layer F.Cu) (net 10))
 (segment (start 78.613 58.928) (end 78.994 58.547) (width 0.79) (layer F.Cu) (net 10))
 (segment (start 78.994 57.658) (end 78.994 60.198) (width 0.79) (layer F.Cu) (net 10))
 (segment (start 78.994 59.309) (end 78.613 58.928) (width 0.79) (layer F.Cu) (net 10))
 (segment (start 78.994 60.198) (end 78.994 59.309) (width 0.79) (layer F.Cu) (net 10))
 (via (at 87.757 54.737) (size 0.8) (drill 0.4) (layers F.Cu B.Cu) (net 10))
 (segment (start 87.6555 54.8385) (end 87.757 54.737) (width 0.79) (layer F.Cu) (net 10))
 (segment (start 86.487 54.8385) (end 87.6555 54.8385) (width 0.79) (layer F.Cu) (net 10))
 (segment (start 86.106 54.737) (end 85.217 55.626) (width 0.79) (layer B.Cu) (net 10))
 (segment (start 87.757 54.737) (end 86.106 54.737) (width 0.79) (layer B.Cu) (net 10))
 (segment (start 81.026 62.23) (end 78.994 60.198) (width 0.79) (layer B.Cu) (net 10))
 (segment (start 85.217 62.23) (end 81.026 62.23) (width 0.79) (layer B.Cu) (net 10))
 (segment (start 86.106 63.119) (end 85.217 62.23) (width 0.79) (layer B.Cu) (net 10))
 (segment (start 87.757 63.119) (end 86.106 63.119) (width 0.79) (layer B.Cu) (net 10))
 (segment (start 81.026 55.626) (end 78.994 57.658) (width 0.79) (layer B.Cu) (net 10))
 (segment (start 85.217 55.626) (end 81.026 55.626) (width 0.79) (layer B.Cu) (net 10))
 (segment (start 89.576 59.578) (end 90.577 60.579) (width 0.35) (layer F.Cu) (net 6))
 (segment (start 86.106 59.578) (end 89.589 59.578) (width 0.35) (layer F.Cu) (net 6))
 (segment (start 86.106 59.578) (end 86.106 59.804) (width 0.35) (layer F.Cu) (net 6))
 (segment (start 86.868 60.579) (end 90.577 60.579) (width 0.35) (layer F.Cu) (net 6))
 (segment (start 86.106 59.804) (end 86.881 60.579) (width 0.35) (layer F.Cu) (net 6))
 (segment (start 86.106 58.039) (end 86.881 57.264) (width 0.35) (layer F.Cu) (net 7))
 (segment (start 86.106 58.054) (end 86.106 58.28) (width 0.35) (layer F.Cu) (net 7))
 (segment (start 89.576 58.278) (end 90.577 57.277) (width 0.35) (layer F.Cu) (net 7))
 (segment (start 86.106 58.278) (end 89.589 58.278) (width 0.35) (layer F.Cu) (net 7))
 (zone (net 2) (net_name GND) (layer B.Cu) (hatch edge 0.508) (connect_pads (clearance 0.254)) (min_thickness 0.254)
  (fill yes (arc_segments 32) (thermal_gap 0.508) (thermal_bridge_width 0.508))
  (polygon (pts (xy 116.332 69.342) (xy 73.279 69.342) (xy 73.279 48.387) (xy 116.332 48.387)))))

